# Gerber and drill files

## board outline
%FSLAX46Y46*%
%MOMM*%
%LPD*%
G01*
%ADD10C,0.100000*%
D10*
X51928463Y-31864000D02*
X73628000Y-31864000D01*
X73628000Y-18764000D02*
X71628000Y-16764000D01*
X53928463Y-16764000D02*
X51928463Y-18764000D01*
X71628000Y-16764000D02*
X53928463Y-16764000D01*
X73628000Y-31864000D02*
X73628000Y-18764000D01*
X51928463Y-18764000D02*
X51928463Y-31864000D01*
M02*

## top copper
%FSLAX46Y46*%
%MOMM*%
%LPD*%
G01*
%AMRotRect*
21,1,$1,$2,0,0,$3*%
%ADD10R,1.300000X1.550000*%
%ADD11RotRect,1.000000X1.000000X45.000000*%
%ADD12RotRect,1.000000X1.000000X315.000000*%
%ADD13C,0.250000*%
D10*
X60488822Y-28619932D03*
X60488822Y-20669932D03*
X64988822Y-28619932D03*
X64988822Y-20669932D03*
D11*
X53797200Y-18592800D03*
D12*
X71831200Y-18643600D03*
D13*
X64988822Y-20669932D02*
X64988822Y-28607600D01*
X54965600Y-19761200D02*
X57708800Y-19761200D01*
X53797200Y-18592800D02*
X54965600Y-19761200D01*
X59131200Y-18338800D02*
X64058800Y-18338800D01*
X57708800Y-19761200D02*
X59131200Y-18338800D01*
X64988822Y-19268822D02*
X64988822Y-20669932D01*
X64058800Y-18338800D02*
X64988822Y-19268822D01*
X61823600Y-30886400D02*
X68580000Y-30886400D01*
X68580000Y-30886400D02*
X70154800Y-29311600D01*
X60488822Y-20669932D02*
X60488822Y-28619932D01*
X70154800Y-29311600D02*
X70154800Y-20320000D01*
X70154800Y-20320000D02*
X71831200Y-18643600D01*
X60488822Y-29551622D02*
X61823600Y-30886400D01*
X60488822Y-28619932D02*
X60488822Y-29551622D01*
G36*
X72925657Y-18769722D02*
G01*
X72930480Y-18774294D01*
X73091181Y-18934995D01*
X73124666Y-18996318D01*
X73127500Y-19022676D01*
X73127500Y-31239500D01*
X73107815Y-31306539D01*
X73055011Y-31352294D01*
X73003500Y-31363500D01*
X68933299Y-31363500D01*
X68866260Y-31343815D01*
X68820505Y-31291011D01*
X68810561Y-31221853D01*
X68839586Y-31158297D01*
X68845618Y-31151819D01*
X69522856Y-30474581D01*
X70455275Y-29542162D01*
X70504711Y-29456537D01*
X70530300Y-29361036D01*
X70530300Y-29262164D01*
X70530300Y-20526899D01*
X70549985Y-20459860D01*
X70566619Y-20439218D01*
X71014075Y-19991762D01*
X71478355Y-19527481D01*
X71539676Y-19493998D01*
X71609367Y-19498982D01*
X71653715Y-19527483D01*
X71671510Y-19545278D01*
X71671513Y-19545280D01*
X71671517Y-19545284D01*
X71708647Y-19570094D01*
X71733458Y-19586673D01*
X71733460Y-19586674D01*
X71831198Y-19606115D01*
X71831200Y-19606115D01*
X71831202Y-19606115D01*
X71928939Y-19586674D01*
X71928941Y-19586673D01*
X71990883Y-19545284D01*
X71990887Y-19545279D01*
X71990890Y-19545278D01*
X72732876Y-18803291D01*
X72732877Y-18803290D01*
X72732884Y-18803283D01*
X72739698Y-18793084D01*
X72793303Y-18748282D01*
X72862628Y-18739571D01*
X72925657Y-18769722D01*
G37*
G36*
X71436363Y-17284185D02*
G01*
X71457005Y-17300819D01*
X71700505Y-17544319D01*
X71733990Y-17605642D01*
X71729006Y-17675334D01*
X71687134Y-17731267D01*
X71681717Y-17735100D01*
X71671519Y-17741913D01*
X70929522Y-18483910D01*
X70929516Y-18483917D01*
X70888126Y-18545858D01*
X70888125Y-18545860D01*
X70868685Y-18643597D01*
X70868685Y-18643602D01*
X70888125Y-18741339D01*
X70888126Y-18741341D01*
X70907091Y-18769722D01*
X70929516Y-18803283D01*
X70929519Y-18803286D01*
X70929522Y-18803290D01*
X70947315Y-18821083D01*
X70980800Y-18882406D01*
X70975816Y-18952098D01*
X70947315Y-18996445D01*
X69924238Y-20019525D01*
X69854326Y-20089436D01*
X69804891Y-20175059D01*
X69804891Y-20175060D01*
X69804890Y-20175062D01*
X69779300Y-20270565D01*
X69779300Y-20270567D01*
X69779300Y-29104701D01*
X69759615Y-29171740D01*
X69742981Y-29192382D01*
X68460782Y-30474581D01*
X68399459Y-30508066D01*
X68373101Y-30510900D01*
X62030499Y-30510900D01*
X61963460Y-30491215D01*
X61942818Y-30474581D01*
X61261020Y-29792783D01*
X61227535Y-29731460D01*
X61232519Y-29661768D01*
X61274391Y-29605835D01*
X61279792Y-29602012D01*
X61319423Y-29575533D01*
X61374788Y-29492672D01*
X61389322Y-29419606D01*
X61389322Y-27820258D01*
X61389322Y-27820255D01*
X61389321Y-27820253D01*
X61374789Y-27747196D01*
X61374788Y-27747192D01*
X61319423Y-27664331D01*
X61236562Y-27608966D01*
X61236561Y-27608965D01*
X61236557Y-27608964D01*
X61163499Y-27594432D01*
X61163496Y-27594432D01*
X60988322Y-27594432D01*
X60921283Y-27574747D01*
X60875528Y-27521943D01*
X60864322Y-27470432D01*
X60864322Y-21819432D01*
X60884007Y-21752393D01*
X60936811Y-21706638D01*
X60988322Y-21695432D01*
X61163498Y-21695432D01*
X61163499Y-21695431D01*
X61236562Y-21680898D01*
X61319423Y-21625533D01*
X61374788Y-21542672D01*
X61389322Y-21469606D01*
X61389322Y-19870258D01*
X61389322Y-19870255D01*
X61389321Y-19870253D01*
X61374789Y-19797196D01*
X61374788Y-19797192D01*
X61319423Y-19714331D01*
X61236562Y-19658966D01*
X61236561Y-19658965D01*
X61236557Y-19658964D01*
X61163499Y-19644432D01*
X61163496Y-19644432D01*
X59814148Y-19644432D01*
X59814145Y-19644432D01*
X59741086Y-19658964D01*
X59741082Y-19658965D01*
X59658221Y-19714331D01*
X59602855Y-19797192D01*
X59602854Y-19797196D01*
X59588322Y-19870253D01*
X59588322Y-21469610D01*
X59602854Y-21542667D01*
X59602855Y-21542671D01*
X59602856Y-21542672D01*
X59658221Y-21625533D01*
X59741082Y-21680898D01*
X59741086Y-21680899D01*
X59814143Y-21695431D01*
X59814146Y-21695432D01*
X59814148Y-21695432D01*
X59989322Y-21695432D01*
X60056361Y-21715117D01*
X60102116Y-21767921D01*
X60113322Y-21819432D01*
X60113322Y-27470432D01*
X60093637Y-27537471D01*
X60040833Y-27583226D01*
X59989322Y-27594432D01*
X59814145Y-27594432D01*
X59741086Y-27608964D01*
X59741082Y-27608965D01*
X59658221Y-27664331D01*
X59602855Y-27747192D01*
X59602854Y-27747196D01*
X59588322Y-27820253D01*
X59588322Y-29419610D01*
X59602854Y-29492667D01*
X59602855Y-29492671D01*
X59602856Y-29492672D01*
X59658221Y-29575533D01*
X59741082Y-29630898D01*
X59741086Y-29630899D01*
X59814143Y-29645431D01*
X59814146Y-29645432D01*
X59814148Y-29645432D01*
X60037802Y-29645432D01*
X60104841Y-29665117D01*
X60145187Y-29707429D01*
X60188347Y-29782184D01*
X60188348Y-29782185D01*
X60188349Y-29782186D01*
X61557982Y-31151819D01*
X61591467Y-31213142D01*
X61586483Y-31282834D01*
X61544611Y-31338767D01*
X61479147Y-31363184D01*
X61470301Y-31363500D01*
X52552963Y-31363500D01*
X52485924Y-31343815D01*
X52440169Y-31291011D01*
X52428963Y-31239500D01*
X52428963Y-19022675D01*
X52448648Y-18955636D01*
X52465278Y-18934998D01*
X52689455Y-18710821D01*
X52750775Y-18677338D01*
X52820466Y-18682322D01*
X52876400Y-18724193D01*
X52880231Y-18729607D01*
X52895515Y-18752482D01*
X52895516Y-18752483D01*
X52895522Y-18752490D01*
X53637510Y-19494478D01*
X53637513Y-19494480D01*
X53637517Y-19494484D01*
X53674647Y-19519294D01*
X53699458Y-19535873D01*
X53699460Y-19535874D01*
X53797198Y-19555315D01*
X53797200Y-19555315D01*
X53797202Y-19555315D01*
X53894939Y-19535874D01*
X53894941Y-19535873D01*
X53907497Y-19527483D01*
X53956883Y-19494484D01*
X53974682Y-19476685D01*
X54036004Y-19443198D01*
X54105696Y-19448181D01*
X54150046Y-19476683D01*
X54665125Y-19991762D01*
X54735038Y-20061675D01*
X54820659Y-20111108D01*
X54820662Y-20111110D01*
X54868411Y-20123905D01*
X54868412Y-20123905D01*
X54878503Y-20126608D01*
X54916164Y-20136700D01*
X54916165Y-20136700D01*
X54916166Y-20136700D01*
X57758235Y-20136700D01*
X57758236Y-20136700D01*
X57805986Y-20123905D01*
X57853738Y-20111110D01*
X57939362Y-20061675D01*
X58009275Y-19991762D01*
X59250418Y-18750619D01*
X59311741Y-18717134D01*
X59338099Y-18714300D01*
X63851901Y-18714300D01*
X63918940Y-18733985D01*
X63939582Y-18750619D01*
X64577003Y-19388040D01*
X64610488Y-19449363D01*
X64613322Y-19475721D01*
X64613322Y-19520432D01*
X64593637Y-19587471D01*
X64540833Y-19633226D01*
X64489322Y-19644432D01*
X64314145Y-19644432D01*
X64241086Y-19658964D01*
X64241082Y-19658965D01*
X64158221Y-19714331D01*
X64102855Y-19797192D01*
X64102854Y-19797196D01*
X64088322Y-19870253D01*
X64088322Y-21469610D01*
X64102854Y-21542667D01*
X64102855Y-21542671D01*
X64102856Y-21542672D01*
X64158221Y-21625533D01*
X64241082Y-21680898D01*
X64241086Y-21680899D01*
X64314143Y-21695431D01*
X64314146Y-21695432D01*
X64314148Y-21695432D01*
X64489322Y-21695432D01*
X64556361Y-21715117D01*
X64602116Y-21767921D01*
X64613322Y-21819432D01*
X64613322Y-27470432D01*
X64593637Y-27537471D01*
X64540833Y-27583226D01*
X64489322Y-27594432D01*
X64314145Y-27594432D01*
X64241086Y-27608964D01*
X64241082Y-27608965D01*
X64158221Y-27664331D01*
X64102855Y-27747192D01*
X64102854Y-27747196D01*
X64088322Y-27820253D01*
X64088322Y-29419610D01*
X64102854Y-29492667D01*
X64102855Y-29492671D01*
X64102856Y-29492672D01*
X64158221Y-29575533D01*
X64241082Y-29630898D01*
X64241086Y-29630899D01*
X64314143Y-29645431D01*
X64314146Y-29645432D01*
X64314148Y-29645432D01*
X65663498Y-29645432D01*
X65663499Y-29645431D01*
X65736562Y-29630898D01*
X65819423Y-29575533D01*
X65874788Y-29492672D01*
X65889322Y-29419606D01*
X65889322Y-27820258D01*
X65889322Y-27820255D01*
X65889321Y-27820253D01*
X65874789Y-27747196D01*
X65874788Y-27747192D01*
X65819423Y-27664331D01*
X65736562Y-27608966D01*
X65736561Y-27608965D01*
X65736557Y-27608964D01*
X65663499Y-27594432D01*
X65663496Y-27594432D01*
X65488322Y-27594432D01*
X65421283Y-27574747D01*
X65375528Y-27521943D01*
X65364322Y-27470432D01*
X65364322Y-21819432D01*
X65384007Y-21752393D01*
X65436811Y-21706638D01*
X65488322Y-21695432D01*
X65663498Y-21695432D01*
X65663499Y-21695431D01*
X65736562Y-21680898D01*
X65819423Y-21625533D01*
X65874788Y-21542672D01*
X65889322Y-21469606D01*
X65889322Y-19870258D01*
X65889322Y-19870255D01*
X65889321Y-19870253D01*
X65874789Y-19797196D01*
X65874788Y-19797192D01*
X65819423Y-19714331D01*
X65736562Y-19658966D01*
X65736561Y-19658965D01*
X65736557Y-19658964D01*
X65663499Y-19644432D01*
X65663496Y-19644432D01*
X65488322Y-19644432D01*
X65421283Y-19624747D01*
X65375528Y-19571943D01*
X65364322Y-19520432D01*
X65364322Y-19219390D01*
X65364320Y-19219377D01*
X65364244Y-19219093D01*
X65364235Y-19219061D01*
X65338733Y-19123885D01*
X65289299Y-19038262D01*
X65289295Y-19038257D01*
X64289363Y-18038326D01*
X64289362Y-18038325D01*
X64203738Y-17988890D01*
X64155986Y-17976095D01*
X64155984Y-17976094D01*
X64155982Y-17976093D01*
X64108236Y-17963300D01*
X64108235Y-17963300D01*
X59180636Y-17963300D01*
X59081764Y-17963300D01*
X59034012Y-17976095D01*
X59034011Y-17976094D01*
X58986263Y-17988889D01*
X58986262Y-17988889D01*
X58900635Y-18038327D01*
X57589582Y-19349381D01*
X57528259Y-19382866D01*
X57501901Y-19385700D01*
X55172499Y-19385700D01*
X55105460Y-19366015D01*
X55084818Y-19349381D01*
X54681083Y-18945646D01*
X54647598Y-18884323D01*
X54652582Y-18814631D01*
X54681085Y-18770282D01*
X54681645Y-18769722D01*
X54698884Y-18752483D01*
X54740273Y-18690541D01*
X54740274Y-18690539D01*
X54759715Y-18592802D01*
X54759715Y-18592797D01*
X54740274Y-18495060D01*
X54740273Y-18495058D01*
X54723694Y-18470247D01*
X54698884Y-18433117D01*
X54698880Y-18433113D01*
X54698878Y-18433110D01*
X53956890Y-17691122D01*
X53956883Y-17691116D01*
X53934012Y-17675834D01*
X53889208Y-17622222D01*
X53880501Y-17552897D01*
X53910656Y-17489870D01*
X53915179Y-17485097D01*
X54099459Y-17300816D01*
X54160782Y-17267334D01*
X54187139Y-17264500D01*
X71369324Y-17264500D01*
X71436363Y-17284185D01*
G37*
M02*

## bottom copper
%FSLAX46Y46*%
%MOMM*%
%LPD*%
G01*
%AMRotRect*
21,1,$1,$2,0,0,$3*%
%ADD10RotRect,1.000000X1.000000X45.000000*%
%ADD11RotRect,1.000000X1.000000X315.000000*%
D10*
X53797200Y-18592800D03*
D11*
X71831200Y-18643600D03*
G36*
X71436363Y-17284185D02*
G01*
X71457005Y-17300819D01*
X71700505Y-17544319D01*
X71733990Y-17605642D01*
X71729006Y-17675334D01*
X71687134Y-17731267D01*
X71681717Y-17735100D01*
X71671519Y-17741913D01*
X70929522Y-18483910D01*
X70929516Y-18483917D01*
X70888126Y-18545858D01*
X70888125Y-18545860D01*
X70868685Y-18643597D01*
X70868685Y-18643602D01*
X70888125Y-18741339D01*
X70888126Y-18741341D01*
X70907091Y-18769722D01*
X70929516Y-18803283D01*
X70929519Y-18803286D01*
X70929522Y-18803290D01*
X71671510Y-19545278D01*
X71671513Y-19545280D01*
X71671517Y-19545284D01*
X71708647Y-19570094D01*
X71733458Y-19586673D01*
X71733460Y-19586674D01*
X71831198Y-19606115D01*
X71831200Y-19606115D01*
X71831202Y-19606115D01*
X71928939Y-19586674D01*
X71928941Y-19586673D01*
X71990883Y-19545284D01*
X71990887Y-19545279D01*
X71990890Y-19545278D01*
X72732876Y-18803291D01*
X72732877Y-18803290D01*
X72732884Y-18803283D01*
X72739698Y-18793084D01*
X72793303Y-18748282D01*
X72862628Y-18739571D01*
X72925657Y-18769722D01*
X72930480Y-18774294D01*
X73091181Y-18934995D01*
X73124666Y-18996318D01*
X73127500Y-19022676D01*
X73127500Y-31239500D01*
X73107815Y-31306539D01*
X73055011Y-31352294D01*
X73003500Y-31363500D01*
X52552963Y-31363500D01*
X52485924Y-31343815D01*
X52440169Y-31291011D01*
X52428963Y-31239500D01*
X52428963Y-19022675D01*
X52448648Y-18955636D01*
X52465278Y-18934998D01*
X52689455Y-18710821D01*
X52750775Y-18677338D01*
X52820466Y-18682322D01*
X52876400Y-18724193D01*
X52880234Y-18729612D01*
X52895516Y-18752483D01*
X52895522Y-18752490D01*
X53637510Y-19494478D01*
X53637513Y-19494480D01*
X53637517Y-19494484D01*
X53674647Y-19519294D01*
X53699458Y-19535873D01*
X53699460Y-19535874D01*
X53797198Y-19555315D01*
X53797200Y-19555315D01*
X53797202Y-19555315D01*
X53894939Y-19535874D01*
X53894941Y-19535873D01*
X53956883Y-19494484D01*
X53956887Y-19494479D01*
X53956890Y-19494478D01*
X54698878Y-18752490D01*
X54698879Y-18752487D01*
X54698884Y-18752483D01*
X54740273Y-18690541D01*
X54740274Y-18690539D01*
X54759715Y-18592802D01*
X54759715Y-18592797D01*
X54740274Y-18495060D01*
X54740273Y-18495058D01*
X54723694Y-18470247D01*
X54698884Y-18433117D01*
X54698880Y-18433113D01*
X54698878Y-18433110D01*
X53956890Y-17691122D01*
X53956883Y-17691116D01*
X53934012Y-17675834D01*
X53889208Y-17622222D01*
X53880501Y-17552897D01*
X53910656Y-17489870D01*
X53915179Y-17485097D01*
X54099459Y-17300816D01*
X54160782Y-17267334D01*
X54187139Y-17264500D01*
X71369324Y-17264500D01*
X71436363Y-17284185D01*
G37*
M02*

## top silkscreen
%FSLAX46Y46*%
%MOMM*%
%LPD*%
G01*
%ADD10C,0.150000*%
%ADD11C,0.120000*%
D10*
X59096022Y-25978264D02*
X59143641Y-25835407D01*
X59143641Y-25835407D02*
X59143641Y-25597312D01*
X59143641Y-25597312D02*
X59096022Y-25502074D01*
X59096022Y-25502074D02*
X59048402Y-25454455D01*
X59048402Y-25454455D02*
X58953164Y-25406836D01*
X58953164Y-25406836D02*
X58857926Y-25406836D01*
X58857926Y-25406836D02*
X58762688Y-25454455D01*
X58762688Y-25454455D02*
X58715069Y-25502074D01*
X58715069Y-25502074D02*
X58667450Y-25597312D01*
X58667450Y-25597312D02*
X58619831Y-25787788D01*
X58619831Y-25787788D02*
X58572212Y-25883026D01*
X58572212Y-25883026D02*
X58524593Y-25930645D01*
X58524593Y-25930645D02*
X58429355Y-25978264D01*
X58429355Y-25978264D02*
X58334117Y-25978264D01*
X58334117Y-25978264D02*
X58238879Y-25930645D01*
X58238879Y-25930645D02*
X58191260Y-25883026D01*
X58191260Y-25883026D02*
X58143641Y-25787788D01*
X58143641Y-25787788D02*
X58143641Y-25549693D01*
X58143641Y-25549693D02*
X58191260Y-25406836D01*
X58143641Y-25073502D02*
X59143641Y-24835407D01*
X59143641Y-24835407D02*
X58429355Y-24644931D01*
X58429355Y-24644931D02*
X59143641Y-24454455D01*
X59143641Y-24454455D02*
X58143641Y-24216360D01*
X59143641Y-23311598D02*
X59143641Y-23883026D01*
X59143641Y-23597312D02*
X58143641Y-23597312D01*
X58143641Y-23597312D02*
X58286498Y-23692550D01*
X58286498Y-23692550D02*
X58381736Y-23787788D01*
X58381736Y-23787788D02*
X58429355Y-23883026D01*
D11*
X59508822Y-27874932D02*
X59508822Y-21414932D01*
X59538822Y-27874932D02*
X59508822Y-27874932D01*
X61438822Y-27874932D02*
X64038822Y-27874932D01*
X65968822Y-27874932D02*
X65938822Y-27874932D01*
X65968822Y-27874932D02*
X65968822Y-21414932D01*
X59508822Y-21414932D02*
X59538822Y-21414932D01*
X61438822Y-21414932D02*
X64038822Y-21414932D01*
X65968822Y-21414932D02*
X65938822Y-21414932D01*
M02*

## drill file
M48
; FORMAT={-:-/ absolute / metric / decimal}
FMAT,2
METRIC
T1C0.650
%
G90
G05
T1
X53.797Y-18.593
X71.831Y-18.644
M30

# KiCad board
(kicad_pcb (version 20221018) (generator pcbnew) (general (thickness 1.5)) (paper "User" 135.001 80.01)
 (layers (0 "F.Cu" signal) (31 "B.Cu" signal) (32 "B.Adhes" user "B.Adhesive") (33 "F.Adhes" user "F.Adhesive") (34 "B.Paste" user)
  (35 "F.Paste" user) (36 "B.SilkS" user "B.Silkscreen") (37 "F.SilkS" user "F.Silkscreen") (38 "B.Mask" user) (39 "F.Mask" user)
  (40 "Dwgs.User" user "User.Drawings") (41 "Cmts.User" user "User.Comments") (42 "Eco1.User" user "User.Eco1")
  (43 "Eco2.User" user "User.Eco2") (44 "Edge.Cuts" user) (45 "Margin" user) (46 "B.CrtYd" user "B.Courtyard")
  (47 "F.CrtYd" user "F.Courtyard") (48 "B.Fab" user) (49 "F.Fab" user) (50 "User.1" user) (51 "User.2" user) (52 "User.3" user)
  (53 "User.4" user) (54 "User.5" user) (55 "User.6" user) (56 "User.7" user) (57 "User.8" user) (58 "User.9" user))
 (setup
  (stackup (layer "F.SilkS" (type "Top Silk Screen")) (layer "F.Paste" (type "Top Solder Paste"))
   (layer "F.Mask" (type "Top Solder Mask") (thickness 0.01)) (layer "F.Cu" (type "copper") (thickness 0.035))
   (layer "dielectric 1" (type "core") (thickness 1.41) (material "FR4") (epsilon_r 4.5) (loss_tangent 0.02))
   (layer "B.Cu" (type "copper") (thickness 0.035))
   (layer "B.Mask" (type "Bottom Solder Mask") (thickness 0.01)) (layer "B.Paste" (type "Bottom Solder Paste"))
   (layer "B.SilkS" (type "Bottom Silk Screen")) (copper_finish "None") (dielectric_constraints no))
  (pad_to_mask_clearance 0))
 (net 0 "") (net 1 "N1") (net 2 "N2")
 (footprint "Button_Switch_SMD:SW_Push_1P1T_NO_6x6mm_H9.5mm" (layer "F.Cu") (at 62.738822 24.644932 90)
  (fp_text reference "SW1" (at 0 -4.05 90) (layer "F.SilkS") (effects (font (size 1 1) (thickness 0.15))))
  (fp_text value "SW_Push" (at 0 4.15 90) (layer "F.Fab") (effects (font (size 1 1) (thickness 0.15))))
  (fp_line (start -3.23 -3.23) (end 3.23 -3.23) (stroke (width 0.12) (type solid)) (layer "F.SilkS"))
  (fp_line (start -3.23 -3.2) (end -3.23 -3.23) (stroke (width 0.12) (type solid)) (layer "F.SilkS"))
  (fp_line (start -3.23 -1.3) (end -3.23 1.3) (stroke (width 0.12) (type solid)) (layer "F.SilkS"))
  (fp_line (start -3.23 3.23) (end -3.23 3.2) (stroke (width 0.12) (type solid)) (layer "F.SilkS"))
  (fp_line (start -3.23 3.23) (end 3.23 3.23) (stroke (width 0.12) (type solid)) (layer "F.SilkS"))
  (fp_line (start 3.23 -3.23) (end 3.23 -3.2) (stroke (width 0.12) (type solid)) (layer "F.SilkS"))
  (fp_line (start 3.23 -1.3) (end 3.23 1.3) (stroke (width 0.12) (type solid)) (layer "F.SilkS"))
  (fp_line (start 3.23 3.23) (end 3.23 3.2) (stroke (width 0.12) (type solid)) (layer "F.SilkS"))
  (pad "1" smd rect (at -3.975 -2.25 90) (size 1.55 1.3) (layers "F.Cu" "F.Paste" "F.Mask") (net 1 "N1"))
  (pad "1" smd rect (at 3.975 -2.25 90) (size 1.55 1.3) (layers "F.Cu" "F.Paste" "F.Mask") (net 1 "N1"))
  (pad "2" smd rect (at -3.975 2.25 90) (size 1.55 1.3) (layers "F.Cu" "F.Paste" "F.Mask") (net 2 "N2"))
  (pad "2" smd rect (at 3.975 2.25 90) (size 1.55 1.3) (layers "F.Cu" "F.Paste" "F.Mask") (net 2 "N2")))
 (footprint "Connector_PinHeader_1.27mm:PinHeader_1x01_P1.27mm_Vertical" (layer "B.Cu") (at 53.7972 18.5928 45)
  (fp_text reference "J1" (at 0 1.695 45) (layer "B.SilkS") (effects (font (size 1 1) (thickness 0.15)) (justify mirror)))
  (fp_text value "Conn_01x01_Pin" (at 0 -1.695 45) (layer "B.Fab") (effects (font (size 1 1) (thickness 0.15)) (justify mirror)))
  (pad "1" thru_hole rect (at 0 0 45) (size 1 1) (drill 0.65) (layers "*.Cu" "*.Mask") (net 2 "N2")))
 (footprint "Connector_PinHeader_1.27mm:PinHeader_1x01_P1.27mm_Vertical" (layer "B.Cu") (at 71.8312 18.6436 -45)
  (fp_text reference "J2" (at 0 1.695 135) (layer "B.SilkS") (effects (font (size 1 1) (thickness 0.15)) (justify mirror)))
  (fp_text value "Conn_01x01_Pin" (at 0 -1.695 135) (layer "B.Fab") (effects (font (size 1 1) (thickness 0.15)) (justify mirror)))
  (pad "1" thru_hole rect (at 0 0 315) (size 1 1) (drill 0.65) (layers "*.Cu" "*.Mask") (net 1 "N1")))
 (gr_line (start 51.928463 31.864) (end 73.628 31.864) (stroke (width 0.1) (type solid)) (layer "Edge.Cuts"))
 (gr_line (start 73.628 18.764) (end 71.628 16.764) (stroke (width 0.1) (type solid)) (layer "Edge.Cuts"))
 (gr_line (start 53.928463 16.764) (end 51.928463 18.764) (stroke (width 0.1) (type solid)) (layer "Edge.Cuts"))
 (gr_line (start 71.628 16.764) (end 53.928463 16.764) (stroke (width 0.1) (type solid)) (layer "Edge.Cuts"))
 (gr_line (start 73.628 31.864) (end 73.628 18.764) (stroke (width 0.1) (type solid)) (layer "Edge.Cuts"))
 (gr_line (start 51.928463 18.764) (end 51.928463 31.864) (stroke (width 0.1) (type solid)) (layer "Edge.Cuts"))
 (segment (start 64.988822 20.669932) (end 64.988822 28.6076) (width 0.25) (layer "F.Cu") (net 2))
 (segment (start 54.9656 19.7612) (end 57.7088 19.7612) (width 0.25) (layer "F.Cu") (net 2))
 (segment (start 53.7972 18.5928) (end 54.9656 19.7612) (width 0.25) (layer "F.Cu") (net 2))
 (segment (start 59.1312 18.3388) (end 64.0588 18.3388) (width 0.25) (layer "F.Cu") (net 2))
 (segment (start 57.7088 19.7612) (end 59.1312 18.3388) (width 0.25) (layer "F.Cu") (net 2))
 (segment (start 64.988822 19.268822) (end 64.988822 20.669932) (width 0.25) (layer "F.Cu") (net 2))
 (segment (start 64.0588 18.3388) (end 64.988822 19.268822) (width 0.25) (layer "F.Cu") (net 2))
 (segment (start 61.8236 30.8864) (end 68.58 30.8864) (width 0.25) (layer "F.Cu") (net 1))
 (segment (start 68.58 30.8864) (end 70.1548 29.3116) (width 0.25) (layer "F.Cu") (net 1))
 (segment (start 60.488822 20.669932) (end 60.488822 28.619932) (width 0.25) (layer "F.Cu") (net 1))
 (segment (start 70.1548 29.3116) (end 70.1548 20.32) (width 0.25) (layer "F.Cu") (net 1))
 (segment (start 70.1548 20.32) (end 71.8312 18.6436) (width 0.25) (layer "F.Cu") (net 1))
 (segment (start 60.488822 29.551622) (end 61.8236 30.8864) (width 0.25) (layer "F.Cu") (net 1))
 (segment (start 60.488822 28.619932) (end 60.488822 29.551622) (width 0.25) (layer "F.Cu") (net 1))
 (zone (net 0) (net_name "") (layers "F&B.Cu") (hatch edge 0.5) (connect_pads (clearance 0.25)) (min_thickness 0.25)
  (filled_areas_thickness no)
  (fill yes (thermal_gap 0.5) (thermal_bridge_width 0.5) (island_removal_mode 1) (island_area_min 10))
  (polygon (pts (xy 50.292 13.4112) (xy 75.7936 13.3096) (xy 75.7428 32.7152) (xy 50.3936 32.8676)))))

